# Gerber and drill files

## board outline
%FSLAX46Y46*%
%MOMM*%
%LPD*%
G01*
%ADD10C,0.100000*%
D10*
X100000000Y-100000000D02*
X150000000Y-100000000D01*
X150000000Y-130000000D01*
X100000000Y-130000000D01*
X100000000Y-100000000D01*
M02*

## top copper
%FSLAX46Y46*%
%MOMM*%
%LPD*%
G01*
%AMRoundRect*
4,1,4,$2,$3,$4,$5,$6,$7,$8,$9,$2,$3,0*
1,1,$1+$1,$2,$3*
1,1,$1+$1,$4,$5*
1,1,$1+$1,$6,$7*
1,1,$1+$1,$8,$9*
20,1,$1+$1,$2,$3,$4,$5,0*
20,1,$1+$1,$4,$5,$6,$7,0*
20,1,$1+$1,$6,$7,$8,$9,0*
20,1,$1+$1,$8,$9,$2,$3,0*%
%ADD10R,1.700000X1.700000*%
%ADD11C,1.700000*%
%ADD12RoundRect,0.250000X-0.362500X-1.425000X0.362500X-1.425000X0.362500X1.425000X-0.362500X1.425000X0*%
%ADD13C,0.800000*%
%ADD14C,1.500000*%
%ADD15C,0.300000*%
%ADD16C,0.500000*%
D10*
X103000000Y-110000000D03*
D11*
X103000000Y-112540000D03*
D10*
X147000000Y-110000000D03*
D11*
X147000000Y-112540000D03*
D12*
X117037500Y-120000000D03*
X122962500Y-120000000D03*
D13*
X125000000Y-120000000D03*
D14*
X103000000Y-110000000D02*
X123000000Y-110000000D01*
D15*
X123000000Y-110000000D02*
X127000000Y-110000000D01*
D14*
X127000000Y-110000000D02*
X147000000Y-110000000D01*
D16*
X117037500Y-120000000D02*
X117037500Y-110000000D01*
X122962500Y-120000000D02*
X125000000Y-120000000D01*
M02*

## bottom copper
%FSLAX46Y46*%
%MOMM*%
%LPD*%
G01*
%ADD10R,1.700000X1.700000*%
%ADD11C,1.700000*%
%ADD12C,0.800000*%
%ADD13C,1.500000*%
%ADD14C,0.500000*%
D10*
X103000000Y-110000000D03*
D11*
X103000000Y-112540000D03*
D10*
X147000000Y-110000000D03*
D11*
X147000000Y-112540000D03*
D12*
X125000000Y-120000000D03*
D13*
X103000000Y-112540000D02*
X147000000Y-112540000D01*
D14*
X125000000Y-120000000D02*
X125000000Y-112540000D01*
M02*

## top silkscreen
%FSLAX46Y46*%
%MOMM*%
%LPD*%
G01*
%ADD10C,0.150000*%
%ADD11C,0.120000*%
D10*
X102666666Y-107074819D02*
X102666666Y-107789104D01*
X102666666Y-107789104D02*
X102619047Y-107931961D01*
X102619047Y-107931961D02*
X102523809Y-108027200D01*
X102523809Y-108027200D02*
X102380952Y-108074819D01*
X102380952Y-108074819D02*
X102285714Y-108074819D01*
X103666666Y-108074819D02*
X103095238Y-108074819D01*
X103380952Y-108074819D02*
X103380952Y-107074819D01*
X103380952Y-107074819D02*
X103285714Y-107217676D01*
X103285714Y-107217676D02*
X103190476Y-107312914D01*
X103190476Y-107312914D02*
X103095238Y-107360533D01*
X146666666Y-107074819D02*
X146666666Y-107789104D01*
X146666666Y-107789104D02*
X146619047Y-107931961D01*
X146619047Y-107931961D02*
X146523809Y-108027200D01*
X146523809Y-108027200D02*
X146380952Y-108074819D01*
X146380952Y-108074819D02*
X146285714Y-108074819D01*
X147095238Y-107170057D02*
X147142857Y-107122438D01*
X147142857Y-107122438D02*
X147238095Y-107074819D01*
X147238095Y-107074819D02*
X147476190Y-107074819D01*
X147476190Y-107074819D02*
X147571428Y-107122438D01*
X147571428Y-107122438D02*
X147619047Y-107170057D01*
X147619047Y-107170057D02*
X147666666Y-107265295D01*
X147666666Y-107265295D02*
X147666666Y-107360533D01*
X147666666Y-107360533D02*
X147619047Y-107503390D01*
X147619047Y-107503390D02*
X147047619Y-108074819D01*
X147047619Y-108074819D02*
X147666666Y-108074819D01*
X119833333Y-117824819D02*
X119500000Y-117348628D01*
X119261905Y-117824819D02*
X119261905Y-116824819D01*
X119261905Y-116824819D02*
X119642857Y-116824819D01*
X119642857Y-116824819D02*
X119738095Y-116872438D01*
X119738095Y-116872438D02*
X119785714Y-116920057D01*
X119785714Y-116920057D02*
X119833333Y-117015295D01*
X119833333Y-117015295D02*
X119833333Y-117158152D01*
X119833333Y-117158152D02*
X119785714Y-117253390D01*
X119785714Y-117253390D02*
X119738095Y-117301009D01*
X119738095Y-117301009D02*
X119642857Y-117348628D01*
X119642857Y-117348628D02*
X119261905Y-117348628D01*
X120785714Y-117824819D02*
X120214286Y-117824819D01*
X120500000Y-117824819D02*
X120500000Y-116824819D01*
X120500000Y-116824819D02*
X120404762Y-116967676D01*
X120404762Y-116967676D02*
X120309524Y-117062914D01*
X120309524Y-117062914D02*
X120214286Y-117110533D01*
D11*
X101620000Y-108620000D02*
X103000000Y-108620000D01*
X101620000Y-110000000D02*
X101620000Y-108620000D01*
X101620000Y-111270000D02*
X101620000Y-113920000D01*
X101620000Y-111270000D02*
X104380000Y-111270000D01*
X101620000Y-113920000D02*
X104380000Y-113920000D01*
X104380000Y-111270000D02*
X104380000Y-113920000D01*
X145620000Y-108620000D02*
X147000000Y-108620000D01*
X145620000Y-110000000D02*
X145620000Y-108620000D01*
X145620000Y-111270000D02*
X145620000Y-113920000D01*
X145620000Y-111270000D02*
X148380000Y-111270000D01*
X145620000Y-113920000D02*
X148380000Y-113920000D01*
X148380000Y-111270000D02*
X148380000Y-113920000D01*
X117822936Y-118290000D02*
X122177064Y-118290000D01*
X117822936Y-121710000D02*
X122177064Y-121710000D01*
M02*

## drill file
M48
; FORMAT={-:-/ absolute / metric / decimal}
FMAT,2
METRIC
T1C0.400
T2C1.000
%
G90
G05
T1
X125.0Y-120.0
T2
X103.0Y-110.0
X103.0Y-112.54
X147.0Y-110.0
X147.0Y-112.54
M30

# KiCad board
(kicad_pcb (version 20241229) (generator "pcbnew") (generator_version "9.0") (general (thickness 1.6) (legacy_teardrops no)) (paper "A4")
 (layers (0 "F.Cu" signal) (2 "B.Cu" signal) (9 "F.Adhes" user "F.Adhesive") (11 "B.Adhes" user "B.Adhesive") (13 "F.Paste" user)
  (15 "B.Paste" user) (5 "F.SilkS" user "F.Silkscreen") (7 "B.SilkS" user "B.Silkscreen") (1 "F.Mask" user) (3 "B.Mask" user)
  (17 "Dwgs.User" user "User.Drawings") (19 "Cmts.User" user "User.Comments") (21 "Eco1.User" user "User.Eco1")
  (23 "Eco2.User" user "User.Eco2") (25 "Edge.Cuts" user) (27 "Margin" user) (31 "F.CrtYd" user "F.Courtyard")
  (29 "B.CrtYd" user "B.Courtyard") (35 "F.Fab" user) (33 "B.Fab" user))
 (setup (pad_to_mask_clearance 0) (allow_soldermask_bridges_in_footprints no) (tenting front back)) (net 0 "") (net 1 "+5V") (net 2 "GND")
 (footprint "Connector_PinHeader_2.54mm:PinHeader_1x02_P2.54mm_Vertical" (layer "F.Cu") (at 103 110)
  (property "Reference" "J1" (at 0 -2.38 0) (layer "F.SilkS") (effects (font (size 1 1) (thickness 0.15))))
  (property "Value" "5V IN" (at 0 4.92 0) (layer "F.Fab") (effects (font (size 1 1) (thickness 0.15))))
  (fp_line (start -1.38 -1.38) (end 0 -1.38) (stroke (width 0.12) (type solid)) (layer "F.SilkS"))
  (fp_line (start -1.38 0) (end -1.38 -1.38) (stroke (width 0.12) (type solid)) (layer "F.SilkS"))
  (fp_line (start -1.38 1.27) (end -1.38 3.92) (stroke (width 0.12) (type solid)) (layer "F.SilkS"))
  (fp_line (start -1.38 1.27) (end 1.38 1.27) (stroke (width 0.12) (type solid)) (layer "F.SilkS"))
  (fp_line (start -1.38 3.92) (end 1.38 3.92) (stroke (width 0.12) (type solid)) (layer "F.SilkS"))
  (fp_line (start 1.38 1.27) (end 1.38 3.92) (stroke (width 0.12) (type solid)) (layer "F.SilkS"))
  (pad "1" thru_hole rect (at 0 0) (size 1.7 1.7) (drill 1) (layers "*.Cu" "*.Mask") (remove_unused_layers no) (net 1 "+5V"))
  (pad "2" thru_hole circle (at 0 2.54) (size 1.7 1.7) (drill 1) (layers "*.Cu" "*.Mask") (remove_unused_layers no) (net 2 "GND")))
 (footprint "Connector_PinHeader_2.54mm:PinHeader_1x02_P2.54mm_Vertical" (layer "F.Cu") (at 147 110)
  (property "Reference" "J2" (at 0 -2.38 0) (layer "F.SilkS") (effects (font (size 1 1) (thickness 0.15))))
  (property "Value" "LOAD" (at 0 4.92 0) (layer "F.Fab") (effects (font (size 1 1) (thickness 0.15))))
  (fp_line (start -1.38 -1.38) (end 0 -1.38) (stroke (width 0.12) (type solid)) (layer "F.SilkS"))
  (fp_line (start -1.38 0) (end -1.38 -1.38) (stroke (width 0.12) (type solid)) (layer "F.SilkS"))
  (fp_line (start -1.38 1.27) (end -1.38 3.92) (stroke (width 0.12) (type solid)) (layer "F.SilkS"))
  (fp_line (start -1.38 1.27) (end 1.38 1.27) (stroke (width 0.12) (type solid)) (layer "F.SilkS"))
  (fp_line (start -1.38 3.92) (end 1.38 3.92) (stroke (width 0.12) (type solid)) (layer "F.SilkS"))
  (fp_line (start 1.38 1.27) (end 1.38 3.92) (stroke (width 0.12) (type solid)) (layer "F.SilkS"))
  (pad "1" thru_hole rect (at 0 0) (size 1.7 1.7) (drill 1) (layers "*.Cu" "*.Mask") (remove_unused_layers no) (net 1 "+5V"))
  (pad "2" thru_hole circle (at 0 2.54) (size 1.7 1.7) (drill 1) (layers "*.Cu" "*.Mask") (remove_unused_layers no) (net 2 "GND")))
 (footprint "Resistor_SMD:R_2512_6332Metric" (layer "F.Cu") (at 120 120)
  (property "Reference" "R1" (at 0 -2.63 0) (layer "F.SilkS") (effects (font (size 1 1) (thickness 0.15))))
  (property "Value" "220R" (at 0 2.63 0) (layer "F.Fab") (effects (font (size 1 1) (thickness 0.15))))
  (fp_line (start -2.177064 -1.71) (end 2.177064 -1.71) (stroke (width 0.12) (type solid)) (layer "F.SilkS"))
  (fp_line (start -2.177064 1.71) (end 2.177064 1.71) (stroke (width 0.12) (type solid)) (layer "F.SilkS"))
  (pad "1" smd roundrect (at -2.9625 0) (size 1.225 3.35) (layers "F.Cu" "F.Mask" "F.Paste") (roundrect_rratio 0.204082) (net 1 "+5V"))
  (pad "2" smd roundrect (at 2.9625 0) (size 1.225 3.35) (layers "F.Cu" "F.Mask" "F.Paste") (roundrect_rratio 0.204082) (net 2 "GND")))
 (gr_rect (start 100 100) (end 150 130) (stroke (width 0.1) (type default)) (fill no) (layer "Edge.Cuts"))
 (segment (start 103 110) (end 123 110) (width 1.5) (layer "F.Cu") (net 1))
 (segment (start 123 110) (end 127 110) (width 0.3) (layer "F.Cu") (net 1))
 (segment (start 127 110) (end 147 110) (width 1.5) (layer "F.Cu") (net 1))
 (segment (start 103 112.54) (end 147 112.54) (width 1.5) (layer "B.Cu") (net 2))
 (segment (start 117.0375 120) (end 117.0375 110) (width 0.5) (layer "F.Cu") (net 1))
 (segment (start 122.9625 120) (end 125 120) (width 0.5) (layer "F.Cu") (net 2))
 (segment (start 125 120) (end 125 112.54) (width 0.5) (layer "B.Cu") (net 2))
 (via (at 125 120) (size 0.8) (drill 0.4) (layers "F.Cu" "B.Cu") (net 2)))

